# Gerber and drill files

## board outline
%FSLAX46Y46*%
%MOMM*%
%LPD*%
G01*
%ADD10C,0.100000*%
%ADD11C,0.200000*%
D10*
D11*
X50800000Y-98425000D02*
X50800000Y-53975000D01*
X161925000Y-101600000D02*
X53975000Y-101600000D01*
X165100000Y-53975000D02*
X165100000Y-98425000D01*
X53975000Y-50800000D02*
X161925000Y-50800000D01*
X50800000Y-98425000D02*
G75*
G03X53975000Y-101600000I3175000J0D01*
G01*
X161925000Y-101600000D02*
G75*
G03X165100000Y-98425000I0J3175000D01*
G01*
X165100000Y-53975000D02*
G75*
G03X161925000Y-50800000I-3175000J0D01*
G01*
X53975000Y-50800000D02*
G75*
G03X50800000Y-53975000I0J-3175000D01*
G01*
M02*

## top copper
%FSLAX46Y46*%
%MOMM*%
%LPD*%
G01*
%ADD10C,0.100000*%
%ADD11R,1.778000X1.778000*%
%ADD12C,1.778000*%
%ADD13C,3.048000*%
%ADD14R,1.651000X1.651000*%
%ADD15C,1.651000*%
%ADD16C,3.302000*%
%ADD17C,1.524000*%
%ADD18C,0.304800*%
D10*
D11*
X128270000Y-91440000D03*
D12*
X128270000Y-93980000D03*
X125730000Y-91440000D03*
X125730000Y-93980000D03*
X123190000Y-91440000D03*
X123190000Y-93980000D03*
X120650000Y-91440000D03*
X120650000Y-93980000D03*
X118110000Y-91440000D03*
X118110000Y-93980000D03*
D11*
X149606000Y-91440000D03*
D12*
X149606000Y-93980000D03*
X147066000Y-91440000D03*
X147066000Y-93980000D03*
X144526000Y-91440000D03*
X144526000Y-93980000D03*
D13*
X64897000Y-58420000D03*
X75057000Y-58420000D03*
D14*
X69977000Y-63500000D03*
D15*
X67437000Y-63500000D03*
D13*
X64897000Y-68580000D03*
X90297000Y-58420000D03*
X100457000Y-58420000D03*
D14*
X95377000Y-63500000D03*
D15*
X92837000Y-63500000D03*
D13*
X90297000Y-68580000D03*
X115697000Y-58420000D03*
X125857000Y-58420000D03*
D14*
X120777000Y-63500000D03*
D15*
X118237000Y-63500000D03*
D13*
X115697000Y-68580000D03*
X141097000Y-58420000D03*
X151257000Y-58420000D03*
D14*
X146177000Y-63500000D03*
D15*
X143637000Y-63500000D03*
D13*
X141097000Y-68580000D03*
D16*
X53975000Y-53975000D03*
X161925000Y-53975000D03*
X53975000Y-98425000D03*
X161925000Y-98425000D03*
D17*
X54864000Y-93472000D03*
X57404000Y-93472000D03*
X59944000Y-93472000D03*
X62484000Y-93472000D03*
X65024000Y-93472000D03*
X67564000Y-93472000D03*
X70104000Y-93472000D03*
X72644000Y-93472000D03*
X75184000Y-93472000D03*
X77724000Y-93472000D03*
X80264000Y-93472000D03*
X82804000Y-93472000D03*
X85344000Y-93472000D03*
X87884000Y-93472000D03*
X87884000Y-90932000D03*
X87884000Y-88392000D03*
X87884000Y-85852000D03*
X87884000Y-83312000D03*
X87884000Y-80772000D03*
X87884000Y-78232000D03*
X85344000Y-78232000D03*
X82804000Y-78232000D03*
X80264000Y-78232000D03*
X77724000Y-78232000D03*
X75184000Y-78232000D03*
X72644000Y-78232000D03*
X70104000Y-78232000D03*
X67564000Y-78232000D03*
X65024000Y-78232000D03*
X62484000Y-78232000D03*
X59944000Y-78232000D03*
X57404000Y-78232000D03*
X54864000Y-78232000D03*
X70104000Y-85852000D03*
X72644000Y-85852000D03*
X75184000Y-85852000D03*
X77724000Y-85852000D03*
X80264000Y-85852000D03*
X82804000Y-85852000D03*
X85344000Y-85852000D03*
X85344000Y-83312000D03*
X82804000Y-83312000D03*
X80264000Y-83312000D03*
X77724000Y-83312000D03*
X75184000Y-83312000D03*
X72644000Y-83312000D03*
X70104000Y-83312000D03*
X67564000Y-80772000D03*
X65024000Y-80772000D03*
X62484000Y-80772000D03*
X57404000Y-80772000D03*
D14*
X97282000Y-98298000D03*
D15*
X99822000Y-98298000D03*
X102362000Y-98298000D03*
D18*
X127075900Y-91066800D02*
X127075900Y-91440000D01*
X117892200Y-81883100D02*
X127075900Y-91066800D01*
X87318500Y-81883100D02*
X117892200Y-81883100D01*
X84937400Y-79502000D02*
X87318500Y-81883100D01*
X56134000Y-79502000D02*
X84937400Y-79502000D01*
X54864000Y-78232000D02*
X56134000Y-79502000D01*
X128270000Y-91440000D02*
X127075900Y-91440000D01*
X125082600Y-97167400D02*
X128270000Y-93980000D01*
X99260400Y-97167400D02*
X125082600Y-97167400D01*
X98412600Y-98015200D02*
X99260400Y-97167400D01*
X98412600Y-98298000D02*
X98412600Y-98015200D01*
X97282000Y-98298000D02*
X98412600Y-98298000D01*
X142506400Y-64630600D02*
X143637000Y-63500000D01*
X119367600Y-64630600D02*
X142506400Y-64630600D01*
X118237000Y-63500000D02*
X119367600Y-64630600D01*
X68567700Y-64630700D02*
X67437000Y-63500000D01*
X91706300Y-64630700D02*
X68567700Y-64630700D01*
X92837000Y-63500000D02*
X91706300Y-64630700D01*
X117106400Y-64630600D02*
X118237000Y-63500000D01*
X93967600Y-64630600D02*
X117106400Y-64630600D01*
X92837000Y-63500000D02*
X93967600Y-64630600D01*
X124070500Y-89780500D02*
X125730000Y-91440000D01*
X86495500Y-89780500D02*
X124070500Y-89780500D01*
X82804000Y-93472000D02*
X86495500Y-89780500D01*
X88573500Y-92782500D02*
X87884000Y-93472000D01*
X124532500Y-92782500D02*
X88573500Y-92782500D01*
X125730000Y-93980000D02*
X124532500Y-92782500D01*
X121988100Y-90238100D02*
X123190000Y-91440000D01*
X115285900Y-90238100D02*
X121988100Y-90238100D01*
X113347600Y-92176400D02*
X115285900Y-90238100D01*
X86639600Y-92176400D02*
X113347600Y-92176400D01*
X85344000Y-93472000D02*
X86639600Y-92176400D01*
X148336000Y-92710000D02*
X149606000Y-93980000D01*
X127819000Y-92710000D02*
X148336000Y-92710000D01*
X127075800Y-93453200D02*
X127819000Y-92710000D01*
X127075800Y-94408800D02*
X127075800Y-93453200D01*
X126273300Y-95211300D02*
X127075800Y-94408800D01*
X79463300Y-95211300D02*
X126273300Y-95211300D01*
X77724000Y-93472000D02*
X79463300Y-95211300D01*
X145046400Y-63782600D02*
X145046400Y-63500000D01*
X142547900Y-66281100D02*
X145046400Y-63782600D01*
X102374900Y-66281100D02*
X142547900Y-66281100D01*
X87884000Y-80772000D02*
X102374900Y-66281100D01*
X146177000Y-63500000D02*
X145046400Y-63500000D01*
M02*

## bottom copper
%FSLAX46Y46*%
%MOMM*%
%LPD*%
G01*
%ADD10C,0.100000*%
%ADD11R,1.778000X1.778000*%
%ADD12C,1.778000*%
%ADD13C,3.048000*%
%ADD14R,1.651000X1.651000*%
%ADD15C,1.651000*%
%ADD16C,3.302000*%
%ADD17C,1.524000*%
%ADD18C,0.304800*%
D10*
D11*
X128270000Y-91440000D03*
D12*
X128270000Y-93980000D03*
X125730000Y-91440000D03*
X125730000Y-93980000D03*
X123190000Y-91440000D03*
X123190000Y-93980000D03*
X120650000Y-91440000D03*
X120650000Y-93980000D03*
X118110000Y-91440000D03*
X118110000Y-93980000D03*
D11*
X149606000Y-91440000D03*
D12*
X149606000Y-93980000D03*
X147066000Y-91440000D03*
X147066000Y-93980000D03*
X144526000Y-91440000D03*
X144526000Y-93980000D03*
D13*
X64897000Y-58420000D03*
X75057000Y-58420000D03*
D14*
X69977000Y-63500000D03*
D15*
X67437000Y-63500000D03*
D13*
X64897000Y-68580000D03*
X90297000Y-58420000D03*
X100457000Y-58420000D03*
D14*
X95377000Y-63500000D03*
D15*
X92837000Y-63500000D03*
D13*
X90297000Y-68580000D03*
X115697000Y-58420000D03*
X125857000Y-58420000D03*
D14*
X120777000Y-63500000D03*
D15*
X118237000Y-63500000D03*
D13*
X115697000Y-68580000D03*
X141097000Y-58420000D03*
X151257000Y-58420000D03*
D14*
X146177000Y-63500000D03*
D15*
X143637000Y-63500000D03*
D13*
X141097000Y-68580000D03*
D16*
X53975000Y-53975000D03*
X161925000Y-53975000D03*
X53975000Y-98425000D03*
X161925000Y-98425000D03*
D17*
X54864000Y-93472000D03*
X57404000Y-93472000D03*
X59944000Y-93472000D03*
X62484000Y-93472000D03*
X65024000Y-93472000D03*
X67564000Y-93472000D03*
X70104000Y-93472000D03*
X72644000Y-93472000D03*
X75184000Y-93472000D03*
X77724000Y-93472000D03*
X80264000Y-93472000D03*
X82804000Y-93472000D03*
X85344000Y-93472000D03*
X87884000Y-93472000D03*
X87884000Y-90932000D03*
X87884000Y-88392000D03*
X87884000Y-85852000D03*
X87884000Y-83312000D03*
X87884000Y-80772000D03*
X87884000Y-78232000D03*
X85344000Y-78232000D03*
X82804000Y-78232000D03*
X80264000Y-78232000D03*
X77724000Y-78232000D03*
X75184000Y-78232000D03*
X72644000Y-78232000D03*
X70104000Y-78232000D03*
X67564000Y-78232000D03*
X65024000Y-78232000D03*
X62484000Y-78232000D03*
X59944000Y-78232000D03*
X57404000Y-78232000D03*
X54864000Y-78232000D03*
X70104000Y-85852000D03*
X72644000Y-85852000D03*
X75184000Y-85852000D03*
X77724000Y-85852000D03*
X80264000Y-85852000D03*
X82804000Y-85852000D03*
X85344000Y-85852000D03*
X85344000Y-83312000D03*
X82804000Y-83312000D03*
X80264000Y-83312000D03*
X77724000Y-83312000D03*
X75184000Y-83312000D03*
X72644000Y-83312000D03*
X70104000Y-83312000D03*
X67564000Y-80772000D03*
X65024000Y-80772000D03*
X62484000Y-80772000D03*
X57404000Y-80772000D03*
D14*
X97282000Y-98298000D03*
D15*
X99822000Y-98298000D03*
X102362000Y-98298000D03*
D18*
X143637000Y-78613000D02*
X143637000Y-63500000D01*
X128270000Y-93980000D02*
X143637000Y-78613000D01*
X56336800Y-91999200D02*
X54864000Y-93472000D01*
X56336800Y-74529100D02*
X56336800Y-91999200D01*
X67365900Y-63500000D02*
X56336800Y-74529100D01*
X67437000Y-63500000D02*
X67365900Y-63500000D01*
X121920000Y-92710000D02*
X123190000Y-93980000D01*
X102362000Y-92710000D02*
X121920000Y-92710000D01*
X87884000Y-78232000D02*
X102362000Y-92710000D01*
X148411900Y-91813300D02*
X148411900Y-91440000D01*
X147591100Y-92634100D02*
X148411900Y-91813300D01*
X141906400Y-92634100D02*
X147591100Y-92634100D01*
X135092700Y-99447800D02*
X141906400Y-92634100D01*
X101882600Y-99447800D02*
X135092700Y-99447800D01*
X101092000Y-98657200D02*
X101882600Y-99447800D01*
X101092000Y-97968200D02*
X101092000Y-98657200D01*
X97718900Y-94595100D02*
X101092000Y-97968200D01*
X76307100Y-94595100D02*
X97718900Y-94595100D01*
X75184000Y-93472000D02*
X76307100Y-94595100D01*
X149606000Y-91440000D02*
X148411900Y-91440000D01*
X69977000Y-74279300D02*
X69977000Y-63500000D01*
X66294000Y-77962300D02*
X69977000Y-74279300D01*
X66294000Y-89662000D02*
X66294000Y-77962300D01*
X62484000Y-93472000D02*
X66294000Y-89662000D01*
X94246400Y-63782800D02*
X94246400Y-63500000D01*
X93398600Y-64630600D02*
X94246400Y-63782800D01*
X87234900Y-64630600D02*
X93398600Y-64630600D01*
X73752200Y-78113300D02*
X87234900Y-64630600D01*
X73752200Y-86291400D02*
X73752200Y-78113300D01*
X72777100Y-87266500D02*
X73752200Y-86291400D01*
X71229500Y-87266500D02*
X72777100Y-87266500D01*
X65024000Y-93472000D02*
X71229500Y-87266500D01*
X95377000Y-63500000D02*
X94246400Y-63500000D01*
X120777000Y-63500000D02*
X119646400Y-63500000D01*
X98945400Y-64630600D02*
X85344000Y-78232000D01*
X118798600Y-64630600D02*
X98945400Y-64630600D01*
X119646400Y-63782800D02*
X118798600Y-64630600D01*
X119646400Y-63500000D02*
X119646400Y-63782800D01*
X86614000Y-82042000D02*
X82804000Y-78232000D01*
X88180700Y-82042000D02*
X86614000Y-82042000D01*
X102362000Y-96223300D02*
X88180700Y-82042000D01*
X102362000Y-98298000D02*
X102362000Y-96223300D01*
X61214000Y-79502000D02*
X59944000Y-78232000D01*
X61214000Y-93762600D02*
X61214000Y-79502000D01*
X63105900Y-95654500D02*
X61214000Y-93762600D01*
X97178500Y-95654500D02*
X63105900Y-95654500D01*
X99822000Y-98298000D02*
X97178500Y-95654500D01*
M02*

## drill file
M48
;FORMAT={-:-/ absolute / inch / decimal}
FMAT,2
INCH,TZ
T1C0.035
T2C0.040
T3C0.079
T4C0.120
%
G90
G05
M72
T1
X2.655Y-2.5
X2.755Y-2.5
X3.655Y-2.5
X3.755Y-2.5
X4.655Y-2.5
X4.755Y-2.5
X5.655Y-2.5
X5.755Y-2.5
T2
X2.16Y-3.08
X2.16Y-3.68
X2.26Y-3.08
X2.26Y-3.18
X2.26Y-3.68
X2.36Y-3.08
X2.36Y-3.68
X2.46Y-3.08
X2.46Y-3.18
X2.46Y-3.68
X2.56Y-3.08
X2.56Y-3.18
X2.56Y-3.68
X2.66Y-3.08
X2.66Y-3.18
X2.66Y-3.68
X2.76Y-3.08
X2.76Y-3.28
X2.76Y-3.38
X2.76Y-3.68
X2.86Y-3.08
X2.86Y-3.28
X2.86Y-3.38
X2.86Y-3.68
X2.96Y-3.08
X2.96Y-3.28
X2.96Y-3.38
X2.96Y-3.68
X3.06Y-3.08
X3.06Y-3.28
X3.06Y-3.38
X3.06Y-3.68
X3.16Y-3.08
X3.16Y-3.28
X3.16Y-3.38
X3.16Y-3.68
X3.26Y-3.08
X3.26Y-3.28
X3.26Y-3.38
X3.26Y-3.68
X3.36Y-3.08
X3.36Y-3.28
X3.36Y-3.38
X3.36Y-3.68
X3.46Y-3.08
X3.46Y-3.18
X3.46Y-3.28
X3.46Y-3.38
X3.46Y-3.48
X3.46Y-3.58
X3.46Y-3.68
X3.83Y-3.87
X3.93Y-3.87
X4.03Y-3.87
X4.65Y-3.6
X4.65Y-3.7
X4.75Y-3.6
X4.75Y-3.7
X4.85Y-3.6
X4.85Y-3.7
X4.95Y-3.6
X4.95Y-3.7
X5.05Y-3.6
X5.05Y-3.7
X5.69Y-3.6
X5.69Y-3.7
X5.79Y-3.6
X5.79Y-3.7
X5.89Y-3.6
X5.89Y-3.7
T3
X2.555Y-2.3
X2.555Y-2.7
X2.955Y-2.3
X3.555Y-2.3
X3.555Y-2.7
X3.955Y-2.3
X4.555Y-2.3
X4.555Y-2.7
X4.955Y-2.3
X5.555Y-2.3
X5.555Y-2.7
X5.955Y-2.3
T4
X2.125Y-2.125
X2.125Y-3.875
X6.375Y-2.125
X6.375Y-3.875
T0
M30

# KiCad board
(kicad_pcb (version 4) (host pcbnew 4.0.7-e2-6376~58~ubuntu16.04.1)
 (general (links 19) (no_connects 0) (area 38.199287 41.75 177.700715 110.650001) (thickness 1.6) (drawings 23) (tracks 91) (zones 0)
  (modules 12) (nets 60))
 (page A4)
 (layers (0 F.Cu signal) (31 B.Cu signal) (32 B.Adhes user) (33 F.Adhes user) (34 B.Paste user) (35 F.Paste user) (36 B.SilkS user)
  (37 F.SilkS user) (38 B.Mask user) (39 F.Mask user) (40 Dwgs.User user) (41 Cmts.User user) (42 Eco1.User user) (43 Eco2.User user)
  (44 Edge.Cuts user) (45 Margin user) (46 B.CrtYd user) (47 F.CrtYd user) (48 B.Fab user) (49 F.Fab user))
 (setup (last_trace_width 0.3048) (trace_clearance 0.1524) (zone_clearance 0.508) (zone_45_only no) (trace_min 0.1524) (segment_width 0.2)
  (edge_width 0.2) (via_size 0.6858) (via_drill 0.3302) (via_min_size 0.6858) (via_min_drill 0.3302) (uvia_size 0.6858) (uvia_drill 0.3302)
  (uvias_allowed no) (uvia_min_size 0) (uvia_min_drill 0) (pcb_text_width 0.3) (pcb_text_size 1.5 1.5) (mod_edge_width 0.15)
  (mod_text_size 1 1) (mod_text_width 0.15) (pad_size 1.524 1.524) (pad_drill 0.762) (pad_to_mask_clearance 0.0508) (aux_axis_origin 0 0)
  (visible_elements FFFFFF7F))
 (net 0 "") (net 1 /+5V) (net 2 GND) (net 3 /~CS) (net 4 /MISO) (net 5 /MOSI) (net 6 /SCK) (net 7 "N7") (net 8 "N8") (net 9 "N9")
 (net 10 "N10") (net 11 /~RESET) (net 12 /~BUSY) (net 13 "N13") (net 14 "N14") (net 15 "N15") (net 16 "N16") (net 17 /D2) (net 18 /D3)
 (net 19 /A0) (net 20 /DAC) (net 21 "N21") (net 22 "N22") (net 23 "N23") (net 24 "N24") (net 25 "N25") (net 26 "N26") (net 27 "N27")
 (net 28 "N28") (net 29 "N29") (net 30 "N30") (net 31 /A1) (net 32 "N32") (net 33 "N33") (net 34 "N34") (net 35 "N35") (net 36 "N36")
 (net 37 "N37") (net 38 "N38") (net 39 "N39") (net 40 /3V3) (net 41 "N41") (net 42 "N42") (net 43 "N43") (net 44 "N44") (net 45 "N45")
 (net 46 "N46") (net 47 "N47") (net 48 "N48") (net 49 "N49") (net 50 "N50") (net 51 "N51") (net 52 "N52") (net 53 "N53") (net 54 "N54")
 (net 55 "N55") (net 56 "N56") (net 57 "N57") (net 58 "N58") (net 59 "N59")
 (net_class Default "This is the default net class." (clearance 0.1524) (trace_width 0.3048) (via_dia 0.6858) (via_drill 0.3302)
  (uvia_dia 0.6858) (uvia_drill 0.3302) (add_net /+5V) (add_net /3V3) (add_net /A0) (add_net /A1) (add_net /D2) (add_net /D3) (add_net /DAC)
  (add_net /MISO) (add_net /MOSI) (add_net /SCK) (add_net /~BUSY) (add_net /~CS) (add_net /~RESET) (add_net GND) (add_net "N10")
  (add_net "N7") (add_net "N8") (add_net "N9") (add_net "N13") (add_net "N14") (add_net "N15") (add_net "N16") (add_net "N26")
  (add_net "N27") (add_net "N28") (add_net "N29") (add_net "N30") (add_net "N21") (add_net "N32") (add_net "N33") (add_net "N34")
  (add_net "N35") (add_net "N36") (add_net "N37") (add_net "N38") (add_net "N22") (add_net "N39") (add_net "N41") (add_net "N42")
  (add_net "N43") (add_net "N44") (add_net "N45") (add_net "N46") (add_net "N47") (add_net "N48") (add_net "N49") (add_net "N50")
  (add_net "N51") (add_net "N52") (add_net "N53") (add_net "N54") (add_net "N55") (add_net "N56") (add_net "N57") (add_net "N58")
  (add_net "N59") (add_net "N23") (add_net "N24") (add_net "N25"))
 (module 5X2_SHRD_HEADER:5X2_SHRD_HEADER (layer F.Cu) (at 123.19 92.71 180)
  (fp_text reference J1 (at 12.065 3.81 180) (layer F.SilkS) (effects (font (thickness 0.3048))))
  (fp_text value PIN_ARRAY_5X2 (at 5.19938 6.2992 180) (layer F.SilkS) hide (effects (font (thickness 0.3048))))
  (pad 1 thru_hole rect (at -5.08 1.27 180) (size 1.778 1.778) (drill 1.016) (layers *.Cu *.Mask F.SilkS) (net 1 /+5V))
  (pad 2 thru_hole circle (at -5.08 -1.27 180) (size 1.778 1.778) (drill 1.016) (layers *.Cu *.Mask F.SilkS) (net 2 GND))
  (pad 3 thru_hole circle (at -2.54 1.27 180) (size 1.778 1.778) (drill 1.016) (layers *.Cu *.Mask F.SilkS) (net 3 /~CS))
  (pad 4 thru_hole circle (at -2.54 -1.27 180) (size 1.778 1.778) (drill 1.016) (layers *.Cu *.Mask F.SilkS) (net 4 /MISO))
  (pad 5 thru_hole circle (at 0 1.27 180) (size 1.778 1.778) (drill 1.016) (layers *.Cu *.Mask F.SilkS) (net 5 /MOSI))
  (pad 6 thru_hole circle (at 0 -1.27 180) (size 1.778 1.778) (drill 1.016) (layers *.Cu *.Mask F.SilkS) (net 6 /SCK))
  (pad 7 thru_hole circle (at 2.54 1.27 180) (size 1.778 1.778) (drill 1.016) (layers *.Cu *.Mask F.SilkS) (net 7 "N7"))
  (pad 8 thru_hole circle (at 2.54 -1.27 180) (size 1.778 1.778) (drill 1.016) (layers *.Cu *.Mask F.SilkS) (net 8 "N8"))
  (pad 9 thru_hole circle (at 5.08 1.27 180) (size 1.778 1.778) (drill 1.016) (layers *.Cu *.Mask F.SilkS) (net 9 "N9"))
  (pad 10 thru_hole circle (at 5.08 -1.27 180) (size 1.778 1.778) (drill 1.016) (layers *.Cu *.Mask F.SilkS) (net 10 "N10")))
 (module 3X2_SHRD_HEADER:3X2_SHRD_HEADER (layer F.Cu) (at 147.066 92.71 180)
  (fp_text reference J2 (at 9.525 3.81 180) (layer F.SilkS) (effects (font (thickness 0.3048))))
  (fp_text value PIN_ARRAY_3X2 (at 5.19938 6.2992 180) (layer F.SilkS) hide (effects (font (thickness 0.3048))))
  (pad 1 thru_hole rect (at -2.54 1.27 180) (size 1.778 1.778) (drill 1.016) (layers *.Cu *.Mask F.SilkS) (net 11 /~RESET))
  (pad 2 thru_hole circle (at -2.54 -1.27 180) (size 1.778 1.778) (drill 1.016) (layers *.Cu *.Mask F.SilkS) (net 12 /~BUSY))
  (pad 3 thru_hole circle (at 0 1.27 180) (size 1.778 1.778) (drill 1.016) (layers *.Cu *.Mask F.SilkS) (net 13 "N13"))
  (pad 4 thru_hole circle (at 0 -1.27 180) (size 1.778 1.778) (drill 1.016) (layers *.Cu *.Mask F.SilkS) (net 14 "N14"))
  (pad 5 thru_hole circle (at 2.54 1.27 180) (size 1.778 1.778) (drill 1.016) (layers *.Cu *.Mask F.SilkS) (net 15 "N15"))
  (pad 6 thru_hole circle (at 2.54 -1.27 180) (size 1.778 1.778) (drill 1.016) (layers *.Cu *.Mask F.SilkS) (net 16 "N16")))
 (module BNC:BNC (layer F.Cu) (at 69.977 58.42)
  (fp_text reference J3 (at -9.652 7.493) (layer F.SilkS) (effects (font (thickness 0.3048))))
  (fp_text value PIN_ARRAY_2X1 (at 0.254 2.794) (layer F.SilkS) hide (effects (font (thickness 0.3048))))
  (pad "" thru_hole circle (at -5.08 0) (size 3.048 3.048) (drill 2.00914) (layers *.Cu *.Mask))
  (pad "" thru_hole circle (at 5.08 0) (size 3.048 3.048) (drill 2.00914) (layers *.Cu *.Mask))
  (pad 1 thru_hole rect (at 0 5.08) (size 1.651 1.651) (drill 0.889) (layers *.Cu *.Mask) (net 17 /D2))
  (pad 2 thru_hole circle (at -2.54 5.08) (size 1.651 1.651) (drill 0.889) (layers *.Cu *.Mask) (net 2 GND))
  (pad "" thru_hole circle (at -5.08 10.16) (size 3.048 3.048) (drill 2.00914) (layers *.Cu *.Mask)))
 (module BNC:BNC (layer F.Cu) (at 95.377 58.42)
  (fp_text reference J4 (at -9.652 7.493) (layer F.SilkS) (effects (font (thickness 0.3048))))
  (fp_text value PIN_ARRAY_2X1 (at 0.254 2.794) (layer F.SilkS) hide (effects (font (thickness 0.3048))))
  (pad "" thru_hole circle (at -5.08 0) (size 3.048 3.048) (drill 2.00914) (layers *.Cu *.Mask))
  (pad "" thru_hole circle (at 5.08 0) (size 3.048 3.048) (drill 2.00914) (layers *.Cu *.Mask))
  (pad 1 thru_hole rect (at 0 5.08) (size 1.651 1.651) (drill 0.889) (layers *.Cu *.Mask) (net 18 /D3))
  (pad 2 thru_hole circle (at -2.54 5.08) (size 1.651 1.651) (drill 0.889) (layers *.Cu *.Mask) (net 2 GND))
  (pad "" thru_hole circle (at -5.08 10.16) (size 3.048 3.048) (drill 2.00914) (layers *.Cu *.Mask)))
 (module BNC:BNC (layer F.Cu) (at 120.777 58.42)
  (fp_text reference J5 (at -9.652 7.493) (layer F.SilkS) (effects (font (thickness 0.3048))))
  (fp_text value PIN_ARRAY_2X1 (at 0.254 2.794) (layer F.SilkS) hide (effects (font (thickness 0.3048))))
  (pad "" thru_hole circle (at -5.08 0) (size 3.048 3.048) (drill 2.00914) (layers *.Cu *.Mask))
  (pad "" thru_hole circle (at 5.08 0) (size 3.048 3.048) (drill 2.00914) (layers *.Cu *.Mask))
  (pad 1 thru_hole rect (at 0 5.08) (size 1.651 1.651) (drill 0.889) (layers *.Cu *.Mask) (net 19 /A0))
  (pad 2 thru_hole circle (at -2.54 5.08) (size 1.651 1.651) (drill 0.889) (layers *.Cu *.Mask) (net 2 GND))
  (pad "" thru_hole circle (at -5.08 10.16) (size 3.048 3.048) (drill 2.00914) (layers *.Cu *.Mask)))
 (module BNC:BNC (layer F.Cu) (at 146.177 58.42)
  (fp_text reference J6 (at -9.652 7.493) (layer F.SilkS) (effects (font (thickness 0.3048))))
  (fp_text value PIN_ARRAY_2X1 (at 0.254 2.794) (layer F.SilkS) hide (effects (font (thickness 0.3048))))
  (pad "" thru_hole circle (at -5.08 0) (size 3.048 3.048) (drill 2.00914) (layers *.Cu *.Mask))
  (pad "" thru_hole circle (at 5.08 0) (size 3.048 3.048) (drill 2.00914) (layers *.Cu *.Mask))
  (pad 1 thru_hole rect (at 0 5.08) (size 1.651 1.651) (drill 0.889) (layers *.Cu *.Mask) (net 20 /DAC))
  (pad 2 thru_hole circle (at -2.54 5.08) (size 1.651 1.651) (drill 0.889) (layers *.Cu *.Mask) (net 2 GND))
  (pad "" thru_hole circle (at -5.08 10.16) (size 3.048 3.048) (drill 2.00914) (layers *.Cu *.Mask)))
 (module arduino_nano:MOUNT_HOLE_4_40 (layer F.Cu) (at 53.975 53.975)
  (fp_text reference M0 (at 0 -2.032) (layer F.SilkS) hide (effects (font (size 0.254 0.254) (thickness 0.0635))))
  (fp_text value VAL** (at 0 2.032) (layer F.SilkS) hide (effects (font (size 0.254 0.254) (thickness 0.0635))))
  (pad "" thru_hole circle (at 0 0) (size 3.302 3.302) (drill 3.048) (layers *.Cu *.SilkS *.Mask)))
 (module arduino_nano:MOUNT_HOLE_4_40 (layer F.Cu) (at 161.925 53.975)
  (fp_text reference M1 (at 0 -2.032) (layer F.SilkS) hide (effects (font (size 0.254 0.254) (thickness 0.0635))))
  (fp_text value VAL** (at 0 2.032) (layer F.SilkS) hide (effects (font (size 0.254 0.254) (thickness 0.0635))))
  (pad "" thru_hole circle (at 0 0) (size 3.302 3.302) (drill 3.048) (layers *.Cu *.SilkS *.Mask)))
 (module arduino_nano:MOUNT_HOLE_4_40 (layer F.Cu) (at 53.975 98.425)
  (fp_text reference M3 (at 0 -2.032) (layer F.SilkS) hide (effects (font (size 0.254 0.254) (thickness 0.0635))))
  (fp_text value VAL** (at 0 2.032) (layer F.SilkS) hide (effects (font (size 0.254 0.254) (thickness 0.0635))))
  (pad "" thru_hole circle (at 0 0) (size 3.302 3.302) (drill 3.048) (layers *.Cu *.SilkS *.Mask)))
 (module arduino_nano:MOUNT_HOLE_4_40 (layer F.Cu) (at 161.925 98.425)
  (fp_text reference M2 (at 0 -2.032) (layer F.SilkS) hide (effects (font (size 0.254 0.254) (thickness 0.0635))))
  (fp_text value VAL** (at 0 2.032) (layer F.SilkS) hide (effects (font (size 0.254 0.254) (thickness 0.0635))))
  (pad "" thru_hole circle (at 0 0) (size 3.302 3.302) (drill 3.048) (layers *.Cu *.SilkS *.Mask)))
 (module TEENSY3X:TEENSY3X (layer F.Cu) (at 71.374 85.852 90)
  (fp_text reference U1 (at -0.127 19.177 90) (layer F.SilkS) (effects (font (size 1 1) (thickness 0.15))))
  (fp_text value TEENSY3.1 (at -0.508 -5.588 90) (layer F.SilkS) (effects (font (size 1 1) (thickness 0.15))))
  (pad 1 thru_hole circle (at -7.62 -16.51 90) (size 1.524 1.524) (drill 1.016) (layers *.Cu *.Mask F.SilkS) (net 2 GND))
  (pad 2 thru_hole circle (at -7.62 -13.97 90) (size 1.524 1.524) (drill 1.016) (layers *.Cu *.Mask F.SilkS) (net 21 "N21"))
  (pad 3 thru_hole circle (at -7.62 -11.43 90) (size 1.524 1.524) (drill 1.016) (layers *.Cu *.Mask F.SilkS) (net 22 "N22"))
  (pad 4 thru_hole circle (at -7.62 -8.89 90) (size 1.524 1.524) (drill 1.016) (layers *.Cu *.Mask F.SilkS) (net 17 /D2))
  (pad 5 thru_hole circle (at -7.62 -6.35 90) (size 1.524 1.524) (drill 1.016) (layers *.Cu *.Mask F.SilkS) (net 18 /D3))
  (pad 6 thru_hole circle (at -7.62 -3.81 90) (size 1.524 1.524) (drill 1.016) (layers *.Cu *.Mask F.SilkS) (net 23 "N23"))
  (pad 7 thru_hole circle (at -7.62 -1.27 90) (size 1.524 1.524) (drill 1.016) (layers *.Cu *.Mask F.SilkS) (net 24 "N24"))
  (pad 8 thru_hole circle (at -7.62 1.27 90) (size 1.524 1.524) (drill 1.016) (layers *.Cu *.Mask F.SilkS) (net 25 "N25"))
  (pad 9 thru_hole circle (at -7.62 3.81 90) (size 1.524 1.524) (drill 1.016) (layers *.Cu *.Mask F.SilkS) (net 11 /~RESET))
  (pad 10 thru_hole circle (at -7.62 6.35 90) (size 1.524 1.524) (drill 1.016) (layers *.Cu *.Mask F.SilkS) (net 12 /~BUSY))
  (pad 11 thru_hole circle (at -7.62 8.89 90) (size 1.524 1.524) (drill 1.016) (layers *.Cu *.Mask F.SilkS) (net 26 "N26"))
  (pad 12 thru_hole circle (at -7.62 11.43 90) (size 1.524 1.524) (drill 1.016) (layers *.Cu *.Mask F.SilkS) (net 3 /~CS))
  (pad 13 thru_hole circle (at -7.62 13.97 90) (size 1.524 1.524) (drill 1.016) (layers *.Cu *.Mask F.SilkS) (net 5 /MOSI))
  (pad 14 thru_hole circle (at -7.62 16.51 90) (size 1.524 1.524) (drill 1.016) (layers *.Cu *.Mask F.SilkS) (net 4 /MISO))
  (pad 15 thru_hole circle (at -5.08 16.51 90) (size 1.524 1.524) (drill 1.016) (layers *.Cu *.Mask F.SilkS) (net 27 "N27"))
  (pad 16 thru_hole circle (at -2.54 16.51 90) (size 1.524 1.524) (drill 1.016) (layers *.Cu *.Mask F.SilkS) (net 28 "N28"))
  (pad 17 thru_hole circle (at 0 16.51 90) (size 1.524 1.524) (drill 1.016) (layers *.Cu *.Mask F.SilkS) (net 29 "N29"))
  (pad 18 thru_hole circle (at 2.54 16.51 90) (size 1.524 1.524) (drill 1.016) (layers *.Cu *.Mask F.SilkS) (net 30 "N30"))
  (pad 19 thru_hole circle (at 5.08 16.51 90) (size 1.524 1.524) (drill 1.016) (layers *.Cu *.Mask F.SilkS) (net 20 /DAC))
  (pad 20 thru_hole circle (at 7.62 16.51 90) (size 1.524 1.524) (drill 1.016) (layers *.Cu *.Mask F.SilkS) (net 6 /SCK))
  (pad 21 thru_hole circle (at 7.62 13.97 90) (size 1.524 1.524) (drill 1.016) (layers *.Cu *.Mask F.SilkS) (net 19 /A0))
  (pad 22 thru_hole circle (at 7.62 11.43 90) (size 1.524 1.524) (drill 1.016) (layers *.Cu *.Mask F.SilkS) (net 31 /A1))
  (pad 23 thru_hole circle (at 7.62 8.89 90) (size 1.524 1.524) (drill 1.016) (layers *.Cu *.Mask F.SilkS) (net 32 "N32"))
  (pad 24 thru_hole circle (at 7.62 6.35 90) (size 1.524 1.524) (drill 1.016) (layers *.Cu *.Mask F.SilkS) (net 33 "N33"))
  (pad 25 thru_hole circle (at 7.62 3.81 90) (size 1.524 1.524) (drill 1.016) (layers *.Cu *.Mask F.SilkS) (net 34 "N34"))
  (pad 26 thru_hole circle (at 7.62 1.27 90) (size 1.524 1.524) (drill 1.016) (layers *.Cu *.Mask F.SilkS) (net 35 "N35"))
  (pad 27 thru_hole circle (at 7.62 -1.27 90) (size 1.524 1.524) (drill 1.016) (layers *.Cu *.Mask F.SilkS) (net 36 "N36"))
  (pad 28 thru_hole circle (at 7.62 -3.81 90) (size 1.524 1.524) (drill 1.016) (layers *.Cu *.Mask F.SilkS) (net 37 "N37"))
  (pad 29 thru_hole circle (at 7.62 -6.35 90) (size 1.524 1.524) (drill 1.016) (layers *.Cu *.Mask F.SilkS) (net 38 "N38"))
  (pad 30 thru_hole circle (at 7.62 -8.89 90) (size 1.524 1.524) (drill 1.016) (layers *.Cu *.Mask F.SilkS) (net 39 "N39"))
  (pad 31 thru_hole circle (at 7.62 -11.43 90) (size 1.524 1.524) (drill 1.016) (layers *.Cu *.Mask F.SilkS) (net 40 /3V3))
  (pad 32 thru_hole circle (at 7.62 -13.97 90) (size 1.524 1.524) (drill 1.016) (layers *.Cu *.Mask F.SilkS) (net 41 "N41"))
  (pad 33 thru_hole circle (at 7.62 -16.51 90) (size 1.524 1.524) (drill 1.016) (layers *.Cu *.Mask F.SilkS) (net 1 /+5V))
  (pad 34 thru_hole circle (at 0 -1.27 90) (size 1.524 1.524) (drill 1.016) (layers *.Cu *.Mask F.SilkS) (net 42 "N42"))
  (pad 35 thru_hole circle (at 0 1.27 90) (size 1.524 1.524) (drill 1.016) (layers *.Cu *.Mask F.SilkS) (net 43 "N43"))
  (pad 36 thru_hole circle (at 0 3.81 90) (size 1.524 1.524) (drill 1.016) (layers *.Cu *.Mask F.SilkS) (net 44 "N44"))
  (pad 37 thru_hole circle (at 0 6.35 90) (size 1.524 1.524) (drill 1.016) (layers *.Cu *.Mask F.SilkS) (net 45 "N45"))
  (pad 38 thru_hole circle (at 0 8.89 90) (size 1.524 1.524) (drill 1.016) (layers *.Cu *.Mask F.SilkS) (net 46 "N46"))
  (pad 39 thru_hole circle (at 0 11.43 90) (size 1.524 1.524) (drill 1.016) (layers *.Cu *.Mask F.SilkS) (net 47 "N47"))
  (pad 40 thru_hole circle (at 0 13.97 90) (size 1.524 1.524) (drill 1.016) (layers *.Cu *.Mask F.SilkS) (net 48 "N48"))
  (pad 41 thru_hole circle (at 2.54 13.97 90) (size 1.524 1.524) (drill 1.016) (layers *.Cu *.Mask F.SilkS) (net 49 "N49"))
  (pad 42 thru_hole circle (at 2.54 11.43 90) (size 1.524 1.524) (drill 1.016) (layers *.Cu *.Mask F.SilkS) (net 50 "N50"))
  (pad 43 thru_hole circle (at 2.54 8.89 90) (size 1.524 1.524) (drill 1.016) (layers *.Cu *.Mask F.SilkS) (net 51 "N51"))
  (pad 44 thru_hole circle (at 2.54 6.35 90) (size 1.524 1.524) (drill 1.016) (layers *.Cu *.Mask F.SilkS) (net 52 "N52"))
  (pad 45 thru_hole circle (at 2.54 3.81 90) (size 1.524 1.524) (drill 1.016) (layers *.Cu *.Mask F.SilkS) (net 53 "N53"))
  (pad 46 thru_hole circle (at 2.54 1.27 90) (size 1.524 1.524) (drill 1.016) (layers *.Cu *.Mask F.SilkS) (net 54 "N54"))
  (pad 47 thru_hole circle (at 2.54 -1.27 90) (size 1.524 1.524) (drill 1.016) (layers *.Cu *.Mask F.SilkS) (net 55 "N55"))
  (pad 48 thru_hole circle (at 5.08 -3.81 90) (size 1.524 1.524) (drill 1.016) (layers *.Cu *.Mask F.SilkS) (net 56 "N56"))
  (pad 49 thru_hole circle (at 5.08 -6.35 90) (size 1.524 1.524) (drill 1.016) (layers *.Cu *.Mask F.SilkS) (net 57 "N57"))
  (pad 50 thru_hole circle (at 5.08 -8.89 90) (size 1.524 1.524) (drill 1.016) (layers *.Cu *.Mask F.SilkS) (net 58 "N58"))
  (pad 51 thru_hole circle (at 5.08 -13.97 90) (size 1.524 1.524) (drill 1.016) (layers *.Cu *.Mask F.SilkS) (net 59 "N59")))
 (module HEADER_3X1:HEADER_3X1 (layer F.Cu) (at 99.822 98.298)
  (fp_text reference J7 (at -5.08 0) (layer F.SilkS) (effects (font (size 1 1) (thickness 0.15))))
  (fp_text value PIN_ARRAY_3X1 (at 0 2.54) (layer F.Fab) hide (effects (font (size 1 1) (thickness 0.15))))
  (pad 1 thru_hole rect (at -2.54 0) (size 1.651 1.651) (drill 1.016) (layers *.Cu *.Mask) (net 2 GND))
  (pad 2 thru_hole circle (at 0 0) (size 1.651 1.651) (drill 1.016) (layers *.Cu *.Mask) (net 40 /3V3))
  (pad 3 thru_hole circle (at 2.54 0) (size 1.651 1.651) (drill 1.016) (layers *.Cu *.Mask) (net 31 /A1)))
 (gr_line (start 50.8 98.425) (end 50.8 53.975) (angle 90) (layer Edge.Cuts) (width 0.2))
 (gr_line (start 161.925 101.6) (end 53.975 101.6) (angle 90) (layer Edge.Cuts) (width 0.2))
 (gr_line (start 165.1 53.975) (end 165.1 98.425) (angle 90) (layer Edge.Cuts) (width 0.2))
 (gr_line (start 53.975 50.8) (end 161.925 50.8) (angle 90) (layer Edge.Cuts) (width 0.2))
 (gr_arc (start 53.975 98.425) (end 53.975 101.6) (angle 90) (layer Edge.Cuts) (width 0.2))
 (gr_arc (start 161.925 98.425) (end 165.1 98.425) (angle 90) (layer Edge.Cuts) (width 0.2))
 (gr_arc (start 161.925 53.975) (end 161.925 50.8) (angle 90) (layer Edge.Cuts) (width 0.2))
 (gr_arc (start 53.975 53.975) (end 50.8 53.975) (angle 90) (layer Edge.Cuts) (width 0.2))
 (segment (start 127.0759 91.0668) (end 127.0759 91.44) (width 0.3048) (layer F.Cu) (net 1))
 (segment (start 117.8922 81.8831) (end 127.0759 91.0668) (width 0.3048) (layer F.Cu) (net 1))
 (segment (start 87.3185 81.8831) (end 117.8922 81.8831) (width 0.3048) (layer F.Cu) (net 1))
 (segment (start 84.9374 79.502) (end 87.3185 81.8831) (width 0.3048) (layer F.Cu) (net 1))
 (segment (start 56.134 79.502) (end 84.9374 79.502) (width 0.3048) (layer F.Cu) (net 1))
 (segment (start 54.864 78.232) (end 56.134 79.502) (width 0.3048) (layer F.Cu) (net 1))
 (segment (start 128.27 91.44) (end 127.0759 91.44) (width 0.3048) (layer F.Cu) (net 1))
 (segment (start 125.0826 97.1674) (end 128.27 93.98) (width 0.3048) (layer F.Cu) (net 2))
 (segment (start 99.2604 97.1674) (end 125.0826 97.1674) (width 0.3048) (layer F.Cu) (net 2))
 (segment (start 98.4126 98.0152) (end 99.2604 97.1674) (width 0.3048) (layer F.Cu) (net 2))
 (segment (start 98.4126 98.298) (end 98.4126 98.0152) (width 0.3048) (layer F.Cu) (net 2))
 (segment (start 97.282 98.298) (end 98.4126 98.298) (width 0.3048) (layer F.Cu) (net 2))
 (segment (start 142.5064 64.6306) (end 143.637 63.5) (width 0.3048) (layer F.Cu) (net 2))
 (segment (start 119.3676 64.6306) (end 142.5064 64.6306) (width 0.3048) (layer F.Cu) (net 2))
 (segment (start 118.237 63.5) (end 119.3676 64.6306) (width 0.3048) (layer F.Cu) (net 2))
 (segment (start 68.5677 64.6307) (end 67.437 63.5) (width 0.3048) (layer F.Cu) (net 2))
 (segment (start 91.7063 64.6307) (end 68.5677 64.6307) (width 0.3048) (layer F.Cu) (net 2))
 (segment (start 92.837 63.5) (end 91.7063 64.6307) (width 0.3048) (layer F.Cu) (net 2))
 (segment (start 117.1064 64.6306) (end 118.237 63.5) (width 0.3048) (layer F.Cu) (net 2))
 (segment (start 93.9676 64.6306) (end 117.1064 64.6306) (width 0.3048) (layer F.Cu) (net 2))
 (segment (start 92.837 63.5) (end 93.9676 64.6306) (width 0.3048) (layer F.Cu) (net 2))
 (segment (start 143.637 78.613) (end 143.637 63.5) (width 0.3048) (layer B.Cu) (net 2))
 (segment (start 128.27 93.98) (end 143.637 78.613) (width 0.3048) (layer B.Cu) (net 2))
 (segment (start 56.3368 91.9992) (end 54.864 93.472) (width 0.3048) (layer B.Cu) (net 2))
 (segment (start 56.3368 74.5291) (end 56.3368 91.9992) (width 0.3048) (layer B.Cu) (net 2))
 (segment (start 67.3659 63.5) (end 56.3368 74.5291) (width 0.3048) (layer B.Cu) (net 2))
 (segment (start 67.437 63.5) (end 67.3659 63.5) (width 0.3048) (layer B.Cu) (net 2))
 (segment (start 124.0705 89.7805) (end 125.73 91.44) (width 0.3048) (layer F.Cu) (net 3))
 (segment (start 86.4955 89.7805) (end 124.0705 89.7805) (width 0.3048) (layer F.Cu) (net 3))
 (segment (start 82.804 93.472) (end 86.4955 89.7805) (width 0.3048) (layer F.Cu) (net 3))
 (segment (start 88.5735 92.7825) (end 87.884 93.472) (width 0.3048) (layer F.Cu) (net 4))
 (segment (start 124.5325 92.7825) (end 88.5735 92.7825) (width 0.3048) (layer F.Cu) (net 4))
 (segment (start 125.73 93.98) (end 124.5325 92.7825) (width 0.3048) (layer F.Cu) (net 4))
 (segment (start 121.9881 90.2381) (end 123.19 91.44) (width 0.3048) (layer F.Cu) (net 5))
 (segment (start 115.2859 90.2381) (end 121.9881 90.2381) (width 0.3048) (layer F.Cu) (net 5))
 (segment (start 113.3476 92.1764) (end 115.2859 90.2381) (width 0.3048) (layer F.Cu) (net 5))
 (segment (start 86.6396 92.1764) (end 113.3476 92.1764) (width 0.3048) (layer F.Cu) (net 5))
 (segment (start 85.344 93.472) (end 86.6396 92.1764) (width 0.3048) (layer F.Cu) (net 5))
 (segment (start 121.92 92.71) (end 123.19 93.98) (width 0.3048) (layer B.Cu) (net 6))
 (segment (start 102.362 92.71) (end 121.92 92.71) (width 0.3048) (layer B.Cu) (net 6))
 (segment (start 87.884 78.232) (end 102.362 92.71) (width 0.3048) (layer B.Cu) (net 6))
 (segment (start 148.4119 91.8133) (end 148.4119 91.44) (width 0.3048) (layer B.Cu) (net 11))
 (segment (start 147.5911 92.6341) (end 148.4119 91.8133) (width 0.3048) (layer B.Cu) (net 11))
 (segment (start 141.9064 92.6341) (end 147.5911 92.6341) (width 0.3048) (layer B.Cu) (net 11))
 (segment (start 135.0927 99.4478) (end 141.9064 92.6341) (width 0.3048) (layer B.Cu) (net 11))
 (segment (start 101.8826 99.4478) (end 135.0927 99.4478) (width 0.3048) (layer B.Cu) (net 11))
 (segment (start 101.092 98.6572) (end 101.8826 99.4478) (width 0.3048) (layer B.Cu) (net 11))
 (segment (start 101.092 97.9682) (end 101.092 98.6572) (width 0.3048) (layer B.Cu) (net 11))
 (segment (start 97.7189 94.5951) (end 101.092 97.9682) (width 0.3048) (layer B.Cu) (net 11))
 (segment (start 76.3071 94.5951) (end 97.7189 94.5951) (width 0.3048) (layer B.Cu) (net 11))
 (segment (start 75.184 93.472) (end 76.3071 94.5951) (width 0.3048) (layer B.Cu) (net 11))
 (segment (start 149.606 91.44) (end 148.4119 91.44) (width 0.3048) (layer B.Cu) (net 11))
 (segment (start 148.336 92.71) (end 149.606 93.98) (width 0.3048) (layer F.Cu) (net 12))
 (segment (start 127.819 92.71) (end 148.336 92.71) (width 0.3048) (layer F.Cu) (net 12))
 (segment (start 127.0758 93.4532) (end 127.819 92.71) (width 0.3048) (layer F.Cu) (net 12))
 (segment (start 127.0758 94.4088) (end 127.0758 93.4532) (width 0.3048) (layer F.Cu) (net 12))
 (segment (start 126.2733 95.2113) (end 127.0758 94.4088) (width 0.3048) (layer F.Cu) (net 12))
 (segment (start 79.4633 95.2113) (end 126.2733 95.2113) (width 0.3048) (layer F.Cu) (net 12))
 (segment (start 77.724 93.472) (end 79.4633 95.2113) (width 0.3048) (layer F.Cu) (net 12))
 (segment (start 69.977 74.2793) (end 69.977 63.5) (width 0.3048) (layer B.Cu) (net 17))
 (segment (start 66.294 77.9623) (end 69.977 74.2793) (width 0.3048) (layer B.Cu) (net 17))
 (segment (start 66.294 89.662) (end 66.294 77.9623) (width 0.3048) (layer B.Cu) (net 17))
 (segment (start 62.484 93.472) (end 66.294 89.662) (width 0.3048) (layer B.Cu) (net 17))
 (segment (start 94.2464 63.7828) (end 94.2464 63.5) (width 0.3048) (layer B.Cu) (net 18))
 (segment (start 93.3986 64.6306) (end 94.2464 63.7828) (width 0.3048) (layer B.Cu) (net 18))
 (segment (start 87.2349 64.6306) (end 93.3986 64.6306) (width 0.3048) (layer B.Cu) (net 18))
 (segment (start 73.7522 78.1133) (end 87.2349 64.6306) (width 0.3048) (layer B.Cu) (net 18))
 (segment (start 73.7522 86.2914) (end 73.7522 78.1133) (width 0.3048) (layer B.Cu) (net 18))
 (segment (start 72.7771 87.2665) (end 73.7522 86.2914) (width 0.3048) (layer B.Cu) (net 18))
 (segment (start 71.2295 87.2665) (end 72.7771 87.2665) (width 0.3048) (layer B.Cu) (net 18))
 (segment (start 65.024 93.472) (end 71.2295 87.2665) (width 0.3048) (layer B.Cu) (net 18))
 (segment (start 95.377 63.5) (end 94.2464 63.5) (width 0.3048) (layer B.Cu) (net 18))
 (segment (start 120.777 63.5) (end 119.6464 63.5) (width 0.3048) (layer B.Cu) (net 19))
 (segment (start 98.9454 64.6306) (end 85.344 78.232) (width 0.3048) (layer B.Cu) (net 19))
 (segment (start 118.7986 64.6306) (end 98.9454 64.6306) (width 0.3048) (layer B.Cu) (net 19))
 (segment (start 119.6464 63.7828) (end 118.7986 64.6306) (width 0.3048) (layer B.Cu) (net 19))
 (segment (start 119.6464 63.5) (end 119.6464 63.7828) (width 0.3048) (layer B.Cu) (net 19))
 (segment (start 145.0464 63.7826) (end 145.0464 63.5) (width 0.3048) (layer F.Cu) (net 20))
 (segment (start 142.5479 66.2811) (end 145.0464 63.7826) (width 0.3048) (layer F.Cu) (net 20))
 (segment (start 102.3749 66.2811) (end 142.5479 66.2811) (width 0.3048) (layer F.Cu) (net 20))
 (segment (start 87.884 80.772) (end 102.3749 66.2811) (width 0.3048) (layer F.Cu) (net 20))
 (segment (start 146.177 63.5) (end 145.0464 63.5) (width 0.3048) (layer F.Cu) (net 20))
 (segment (start 86.614 82.042) (end 82.804 78.232) (width 0.3048) (layer B.Cu) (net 31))
 (segment (start 88.1807 82.042) (end 86.614 82.042) (width 0.3048) (layer B.Cu) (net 31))
 (segment (start 102.362 96.2233) (end 88.1807 82.042) (width 0.3048) (layer B.Cu) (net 31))
 (segment (start 102.362 98.298) (end 102.362 96.2233) (width 0.3048) (layer B.Cu) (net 31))
 (segment (start 61.214 79.502) (end 59.944 78.232) (width 0.3048) (layer B.Cu) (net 40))
 (segment (start 61.214 93.7626) (end 61.214 79.502) (width 0.3048) (layer B.Cu) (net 40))
 (segment (start 63.1059 95.6545) (end 61.214 93.7626) (width 0.3048) (layer B.Cu) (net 40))
 (segment (start 97.1785 95.6545) (end 63.1059 95.6545) (width 0.3048) (layer B.Cu) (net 40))
 (segment (start 99.822 98.298) (end 97.1785 95.6545) (width 0.3048) (layer B.Cu) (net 40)))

